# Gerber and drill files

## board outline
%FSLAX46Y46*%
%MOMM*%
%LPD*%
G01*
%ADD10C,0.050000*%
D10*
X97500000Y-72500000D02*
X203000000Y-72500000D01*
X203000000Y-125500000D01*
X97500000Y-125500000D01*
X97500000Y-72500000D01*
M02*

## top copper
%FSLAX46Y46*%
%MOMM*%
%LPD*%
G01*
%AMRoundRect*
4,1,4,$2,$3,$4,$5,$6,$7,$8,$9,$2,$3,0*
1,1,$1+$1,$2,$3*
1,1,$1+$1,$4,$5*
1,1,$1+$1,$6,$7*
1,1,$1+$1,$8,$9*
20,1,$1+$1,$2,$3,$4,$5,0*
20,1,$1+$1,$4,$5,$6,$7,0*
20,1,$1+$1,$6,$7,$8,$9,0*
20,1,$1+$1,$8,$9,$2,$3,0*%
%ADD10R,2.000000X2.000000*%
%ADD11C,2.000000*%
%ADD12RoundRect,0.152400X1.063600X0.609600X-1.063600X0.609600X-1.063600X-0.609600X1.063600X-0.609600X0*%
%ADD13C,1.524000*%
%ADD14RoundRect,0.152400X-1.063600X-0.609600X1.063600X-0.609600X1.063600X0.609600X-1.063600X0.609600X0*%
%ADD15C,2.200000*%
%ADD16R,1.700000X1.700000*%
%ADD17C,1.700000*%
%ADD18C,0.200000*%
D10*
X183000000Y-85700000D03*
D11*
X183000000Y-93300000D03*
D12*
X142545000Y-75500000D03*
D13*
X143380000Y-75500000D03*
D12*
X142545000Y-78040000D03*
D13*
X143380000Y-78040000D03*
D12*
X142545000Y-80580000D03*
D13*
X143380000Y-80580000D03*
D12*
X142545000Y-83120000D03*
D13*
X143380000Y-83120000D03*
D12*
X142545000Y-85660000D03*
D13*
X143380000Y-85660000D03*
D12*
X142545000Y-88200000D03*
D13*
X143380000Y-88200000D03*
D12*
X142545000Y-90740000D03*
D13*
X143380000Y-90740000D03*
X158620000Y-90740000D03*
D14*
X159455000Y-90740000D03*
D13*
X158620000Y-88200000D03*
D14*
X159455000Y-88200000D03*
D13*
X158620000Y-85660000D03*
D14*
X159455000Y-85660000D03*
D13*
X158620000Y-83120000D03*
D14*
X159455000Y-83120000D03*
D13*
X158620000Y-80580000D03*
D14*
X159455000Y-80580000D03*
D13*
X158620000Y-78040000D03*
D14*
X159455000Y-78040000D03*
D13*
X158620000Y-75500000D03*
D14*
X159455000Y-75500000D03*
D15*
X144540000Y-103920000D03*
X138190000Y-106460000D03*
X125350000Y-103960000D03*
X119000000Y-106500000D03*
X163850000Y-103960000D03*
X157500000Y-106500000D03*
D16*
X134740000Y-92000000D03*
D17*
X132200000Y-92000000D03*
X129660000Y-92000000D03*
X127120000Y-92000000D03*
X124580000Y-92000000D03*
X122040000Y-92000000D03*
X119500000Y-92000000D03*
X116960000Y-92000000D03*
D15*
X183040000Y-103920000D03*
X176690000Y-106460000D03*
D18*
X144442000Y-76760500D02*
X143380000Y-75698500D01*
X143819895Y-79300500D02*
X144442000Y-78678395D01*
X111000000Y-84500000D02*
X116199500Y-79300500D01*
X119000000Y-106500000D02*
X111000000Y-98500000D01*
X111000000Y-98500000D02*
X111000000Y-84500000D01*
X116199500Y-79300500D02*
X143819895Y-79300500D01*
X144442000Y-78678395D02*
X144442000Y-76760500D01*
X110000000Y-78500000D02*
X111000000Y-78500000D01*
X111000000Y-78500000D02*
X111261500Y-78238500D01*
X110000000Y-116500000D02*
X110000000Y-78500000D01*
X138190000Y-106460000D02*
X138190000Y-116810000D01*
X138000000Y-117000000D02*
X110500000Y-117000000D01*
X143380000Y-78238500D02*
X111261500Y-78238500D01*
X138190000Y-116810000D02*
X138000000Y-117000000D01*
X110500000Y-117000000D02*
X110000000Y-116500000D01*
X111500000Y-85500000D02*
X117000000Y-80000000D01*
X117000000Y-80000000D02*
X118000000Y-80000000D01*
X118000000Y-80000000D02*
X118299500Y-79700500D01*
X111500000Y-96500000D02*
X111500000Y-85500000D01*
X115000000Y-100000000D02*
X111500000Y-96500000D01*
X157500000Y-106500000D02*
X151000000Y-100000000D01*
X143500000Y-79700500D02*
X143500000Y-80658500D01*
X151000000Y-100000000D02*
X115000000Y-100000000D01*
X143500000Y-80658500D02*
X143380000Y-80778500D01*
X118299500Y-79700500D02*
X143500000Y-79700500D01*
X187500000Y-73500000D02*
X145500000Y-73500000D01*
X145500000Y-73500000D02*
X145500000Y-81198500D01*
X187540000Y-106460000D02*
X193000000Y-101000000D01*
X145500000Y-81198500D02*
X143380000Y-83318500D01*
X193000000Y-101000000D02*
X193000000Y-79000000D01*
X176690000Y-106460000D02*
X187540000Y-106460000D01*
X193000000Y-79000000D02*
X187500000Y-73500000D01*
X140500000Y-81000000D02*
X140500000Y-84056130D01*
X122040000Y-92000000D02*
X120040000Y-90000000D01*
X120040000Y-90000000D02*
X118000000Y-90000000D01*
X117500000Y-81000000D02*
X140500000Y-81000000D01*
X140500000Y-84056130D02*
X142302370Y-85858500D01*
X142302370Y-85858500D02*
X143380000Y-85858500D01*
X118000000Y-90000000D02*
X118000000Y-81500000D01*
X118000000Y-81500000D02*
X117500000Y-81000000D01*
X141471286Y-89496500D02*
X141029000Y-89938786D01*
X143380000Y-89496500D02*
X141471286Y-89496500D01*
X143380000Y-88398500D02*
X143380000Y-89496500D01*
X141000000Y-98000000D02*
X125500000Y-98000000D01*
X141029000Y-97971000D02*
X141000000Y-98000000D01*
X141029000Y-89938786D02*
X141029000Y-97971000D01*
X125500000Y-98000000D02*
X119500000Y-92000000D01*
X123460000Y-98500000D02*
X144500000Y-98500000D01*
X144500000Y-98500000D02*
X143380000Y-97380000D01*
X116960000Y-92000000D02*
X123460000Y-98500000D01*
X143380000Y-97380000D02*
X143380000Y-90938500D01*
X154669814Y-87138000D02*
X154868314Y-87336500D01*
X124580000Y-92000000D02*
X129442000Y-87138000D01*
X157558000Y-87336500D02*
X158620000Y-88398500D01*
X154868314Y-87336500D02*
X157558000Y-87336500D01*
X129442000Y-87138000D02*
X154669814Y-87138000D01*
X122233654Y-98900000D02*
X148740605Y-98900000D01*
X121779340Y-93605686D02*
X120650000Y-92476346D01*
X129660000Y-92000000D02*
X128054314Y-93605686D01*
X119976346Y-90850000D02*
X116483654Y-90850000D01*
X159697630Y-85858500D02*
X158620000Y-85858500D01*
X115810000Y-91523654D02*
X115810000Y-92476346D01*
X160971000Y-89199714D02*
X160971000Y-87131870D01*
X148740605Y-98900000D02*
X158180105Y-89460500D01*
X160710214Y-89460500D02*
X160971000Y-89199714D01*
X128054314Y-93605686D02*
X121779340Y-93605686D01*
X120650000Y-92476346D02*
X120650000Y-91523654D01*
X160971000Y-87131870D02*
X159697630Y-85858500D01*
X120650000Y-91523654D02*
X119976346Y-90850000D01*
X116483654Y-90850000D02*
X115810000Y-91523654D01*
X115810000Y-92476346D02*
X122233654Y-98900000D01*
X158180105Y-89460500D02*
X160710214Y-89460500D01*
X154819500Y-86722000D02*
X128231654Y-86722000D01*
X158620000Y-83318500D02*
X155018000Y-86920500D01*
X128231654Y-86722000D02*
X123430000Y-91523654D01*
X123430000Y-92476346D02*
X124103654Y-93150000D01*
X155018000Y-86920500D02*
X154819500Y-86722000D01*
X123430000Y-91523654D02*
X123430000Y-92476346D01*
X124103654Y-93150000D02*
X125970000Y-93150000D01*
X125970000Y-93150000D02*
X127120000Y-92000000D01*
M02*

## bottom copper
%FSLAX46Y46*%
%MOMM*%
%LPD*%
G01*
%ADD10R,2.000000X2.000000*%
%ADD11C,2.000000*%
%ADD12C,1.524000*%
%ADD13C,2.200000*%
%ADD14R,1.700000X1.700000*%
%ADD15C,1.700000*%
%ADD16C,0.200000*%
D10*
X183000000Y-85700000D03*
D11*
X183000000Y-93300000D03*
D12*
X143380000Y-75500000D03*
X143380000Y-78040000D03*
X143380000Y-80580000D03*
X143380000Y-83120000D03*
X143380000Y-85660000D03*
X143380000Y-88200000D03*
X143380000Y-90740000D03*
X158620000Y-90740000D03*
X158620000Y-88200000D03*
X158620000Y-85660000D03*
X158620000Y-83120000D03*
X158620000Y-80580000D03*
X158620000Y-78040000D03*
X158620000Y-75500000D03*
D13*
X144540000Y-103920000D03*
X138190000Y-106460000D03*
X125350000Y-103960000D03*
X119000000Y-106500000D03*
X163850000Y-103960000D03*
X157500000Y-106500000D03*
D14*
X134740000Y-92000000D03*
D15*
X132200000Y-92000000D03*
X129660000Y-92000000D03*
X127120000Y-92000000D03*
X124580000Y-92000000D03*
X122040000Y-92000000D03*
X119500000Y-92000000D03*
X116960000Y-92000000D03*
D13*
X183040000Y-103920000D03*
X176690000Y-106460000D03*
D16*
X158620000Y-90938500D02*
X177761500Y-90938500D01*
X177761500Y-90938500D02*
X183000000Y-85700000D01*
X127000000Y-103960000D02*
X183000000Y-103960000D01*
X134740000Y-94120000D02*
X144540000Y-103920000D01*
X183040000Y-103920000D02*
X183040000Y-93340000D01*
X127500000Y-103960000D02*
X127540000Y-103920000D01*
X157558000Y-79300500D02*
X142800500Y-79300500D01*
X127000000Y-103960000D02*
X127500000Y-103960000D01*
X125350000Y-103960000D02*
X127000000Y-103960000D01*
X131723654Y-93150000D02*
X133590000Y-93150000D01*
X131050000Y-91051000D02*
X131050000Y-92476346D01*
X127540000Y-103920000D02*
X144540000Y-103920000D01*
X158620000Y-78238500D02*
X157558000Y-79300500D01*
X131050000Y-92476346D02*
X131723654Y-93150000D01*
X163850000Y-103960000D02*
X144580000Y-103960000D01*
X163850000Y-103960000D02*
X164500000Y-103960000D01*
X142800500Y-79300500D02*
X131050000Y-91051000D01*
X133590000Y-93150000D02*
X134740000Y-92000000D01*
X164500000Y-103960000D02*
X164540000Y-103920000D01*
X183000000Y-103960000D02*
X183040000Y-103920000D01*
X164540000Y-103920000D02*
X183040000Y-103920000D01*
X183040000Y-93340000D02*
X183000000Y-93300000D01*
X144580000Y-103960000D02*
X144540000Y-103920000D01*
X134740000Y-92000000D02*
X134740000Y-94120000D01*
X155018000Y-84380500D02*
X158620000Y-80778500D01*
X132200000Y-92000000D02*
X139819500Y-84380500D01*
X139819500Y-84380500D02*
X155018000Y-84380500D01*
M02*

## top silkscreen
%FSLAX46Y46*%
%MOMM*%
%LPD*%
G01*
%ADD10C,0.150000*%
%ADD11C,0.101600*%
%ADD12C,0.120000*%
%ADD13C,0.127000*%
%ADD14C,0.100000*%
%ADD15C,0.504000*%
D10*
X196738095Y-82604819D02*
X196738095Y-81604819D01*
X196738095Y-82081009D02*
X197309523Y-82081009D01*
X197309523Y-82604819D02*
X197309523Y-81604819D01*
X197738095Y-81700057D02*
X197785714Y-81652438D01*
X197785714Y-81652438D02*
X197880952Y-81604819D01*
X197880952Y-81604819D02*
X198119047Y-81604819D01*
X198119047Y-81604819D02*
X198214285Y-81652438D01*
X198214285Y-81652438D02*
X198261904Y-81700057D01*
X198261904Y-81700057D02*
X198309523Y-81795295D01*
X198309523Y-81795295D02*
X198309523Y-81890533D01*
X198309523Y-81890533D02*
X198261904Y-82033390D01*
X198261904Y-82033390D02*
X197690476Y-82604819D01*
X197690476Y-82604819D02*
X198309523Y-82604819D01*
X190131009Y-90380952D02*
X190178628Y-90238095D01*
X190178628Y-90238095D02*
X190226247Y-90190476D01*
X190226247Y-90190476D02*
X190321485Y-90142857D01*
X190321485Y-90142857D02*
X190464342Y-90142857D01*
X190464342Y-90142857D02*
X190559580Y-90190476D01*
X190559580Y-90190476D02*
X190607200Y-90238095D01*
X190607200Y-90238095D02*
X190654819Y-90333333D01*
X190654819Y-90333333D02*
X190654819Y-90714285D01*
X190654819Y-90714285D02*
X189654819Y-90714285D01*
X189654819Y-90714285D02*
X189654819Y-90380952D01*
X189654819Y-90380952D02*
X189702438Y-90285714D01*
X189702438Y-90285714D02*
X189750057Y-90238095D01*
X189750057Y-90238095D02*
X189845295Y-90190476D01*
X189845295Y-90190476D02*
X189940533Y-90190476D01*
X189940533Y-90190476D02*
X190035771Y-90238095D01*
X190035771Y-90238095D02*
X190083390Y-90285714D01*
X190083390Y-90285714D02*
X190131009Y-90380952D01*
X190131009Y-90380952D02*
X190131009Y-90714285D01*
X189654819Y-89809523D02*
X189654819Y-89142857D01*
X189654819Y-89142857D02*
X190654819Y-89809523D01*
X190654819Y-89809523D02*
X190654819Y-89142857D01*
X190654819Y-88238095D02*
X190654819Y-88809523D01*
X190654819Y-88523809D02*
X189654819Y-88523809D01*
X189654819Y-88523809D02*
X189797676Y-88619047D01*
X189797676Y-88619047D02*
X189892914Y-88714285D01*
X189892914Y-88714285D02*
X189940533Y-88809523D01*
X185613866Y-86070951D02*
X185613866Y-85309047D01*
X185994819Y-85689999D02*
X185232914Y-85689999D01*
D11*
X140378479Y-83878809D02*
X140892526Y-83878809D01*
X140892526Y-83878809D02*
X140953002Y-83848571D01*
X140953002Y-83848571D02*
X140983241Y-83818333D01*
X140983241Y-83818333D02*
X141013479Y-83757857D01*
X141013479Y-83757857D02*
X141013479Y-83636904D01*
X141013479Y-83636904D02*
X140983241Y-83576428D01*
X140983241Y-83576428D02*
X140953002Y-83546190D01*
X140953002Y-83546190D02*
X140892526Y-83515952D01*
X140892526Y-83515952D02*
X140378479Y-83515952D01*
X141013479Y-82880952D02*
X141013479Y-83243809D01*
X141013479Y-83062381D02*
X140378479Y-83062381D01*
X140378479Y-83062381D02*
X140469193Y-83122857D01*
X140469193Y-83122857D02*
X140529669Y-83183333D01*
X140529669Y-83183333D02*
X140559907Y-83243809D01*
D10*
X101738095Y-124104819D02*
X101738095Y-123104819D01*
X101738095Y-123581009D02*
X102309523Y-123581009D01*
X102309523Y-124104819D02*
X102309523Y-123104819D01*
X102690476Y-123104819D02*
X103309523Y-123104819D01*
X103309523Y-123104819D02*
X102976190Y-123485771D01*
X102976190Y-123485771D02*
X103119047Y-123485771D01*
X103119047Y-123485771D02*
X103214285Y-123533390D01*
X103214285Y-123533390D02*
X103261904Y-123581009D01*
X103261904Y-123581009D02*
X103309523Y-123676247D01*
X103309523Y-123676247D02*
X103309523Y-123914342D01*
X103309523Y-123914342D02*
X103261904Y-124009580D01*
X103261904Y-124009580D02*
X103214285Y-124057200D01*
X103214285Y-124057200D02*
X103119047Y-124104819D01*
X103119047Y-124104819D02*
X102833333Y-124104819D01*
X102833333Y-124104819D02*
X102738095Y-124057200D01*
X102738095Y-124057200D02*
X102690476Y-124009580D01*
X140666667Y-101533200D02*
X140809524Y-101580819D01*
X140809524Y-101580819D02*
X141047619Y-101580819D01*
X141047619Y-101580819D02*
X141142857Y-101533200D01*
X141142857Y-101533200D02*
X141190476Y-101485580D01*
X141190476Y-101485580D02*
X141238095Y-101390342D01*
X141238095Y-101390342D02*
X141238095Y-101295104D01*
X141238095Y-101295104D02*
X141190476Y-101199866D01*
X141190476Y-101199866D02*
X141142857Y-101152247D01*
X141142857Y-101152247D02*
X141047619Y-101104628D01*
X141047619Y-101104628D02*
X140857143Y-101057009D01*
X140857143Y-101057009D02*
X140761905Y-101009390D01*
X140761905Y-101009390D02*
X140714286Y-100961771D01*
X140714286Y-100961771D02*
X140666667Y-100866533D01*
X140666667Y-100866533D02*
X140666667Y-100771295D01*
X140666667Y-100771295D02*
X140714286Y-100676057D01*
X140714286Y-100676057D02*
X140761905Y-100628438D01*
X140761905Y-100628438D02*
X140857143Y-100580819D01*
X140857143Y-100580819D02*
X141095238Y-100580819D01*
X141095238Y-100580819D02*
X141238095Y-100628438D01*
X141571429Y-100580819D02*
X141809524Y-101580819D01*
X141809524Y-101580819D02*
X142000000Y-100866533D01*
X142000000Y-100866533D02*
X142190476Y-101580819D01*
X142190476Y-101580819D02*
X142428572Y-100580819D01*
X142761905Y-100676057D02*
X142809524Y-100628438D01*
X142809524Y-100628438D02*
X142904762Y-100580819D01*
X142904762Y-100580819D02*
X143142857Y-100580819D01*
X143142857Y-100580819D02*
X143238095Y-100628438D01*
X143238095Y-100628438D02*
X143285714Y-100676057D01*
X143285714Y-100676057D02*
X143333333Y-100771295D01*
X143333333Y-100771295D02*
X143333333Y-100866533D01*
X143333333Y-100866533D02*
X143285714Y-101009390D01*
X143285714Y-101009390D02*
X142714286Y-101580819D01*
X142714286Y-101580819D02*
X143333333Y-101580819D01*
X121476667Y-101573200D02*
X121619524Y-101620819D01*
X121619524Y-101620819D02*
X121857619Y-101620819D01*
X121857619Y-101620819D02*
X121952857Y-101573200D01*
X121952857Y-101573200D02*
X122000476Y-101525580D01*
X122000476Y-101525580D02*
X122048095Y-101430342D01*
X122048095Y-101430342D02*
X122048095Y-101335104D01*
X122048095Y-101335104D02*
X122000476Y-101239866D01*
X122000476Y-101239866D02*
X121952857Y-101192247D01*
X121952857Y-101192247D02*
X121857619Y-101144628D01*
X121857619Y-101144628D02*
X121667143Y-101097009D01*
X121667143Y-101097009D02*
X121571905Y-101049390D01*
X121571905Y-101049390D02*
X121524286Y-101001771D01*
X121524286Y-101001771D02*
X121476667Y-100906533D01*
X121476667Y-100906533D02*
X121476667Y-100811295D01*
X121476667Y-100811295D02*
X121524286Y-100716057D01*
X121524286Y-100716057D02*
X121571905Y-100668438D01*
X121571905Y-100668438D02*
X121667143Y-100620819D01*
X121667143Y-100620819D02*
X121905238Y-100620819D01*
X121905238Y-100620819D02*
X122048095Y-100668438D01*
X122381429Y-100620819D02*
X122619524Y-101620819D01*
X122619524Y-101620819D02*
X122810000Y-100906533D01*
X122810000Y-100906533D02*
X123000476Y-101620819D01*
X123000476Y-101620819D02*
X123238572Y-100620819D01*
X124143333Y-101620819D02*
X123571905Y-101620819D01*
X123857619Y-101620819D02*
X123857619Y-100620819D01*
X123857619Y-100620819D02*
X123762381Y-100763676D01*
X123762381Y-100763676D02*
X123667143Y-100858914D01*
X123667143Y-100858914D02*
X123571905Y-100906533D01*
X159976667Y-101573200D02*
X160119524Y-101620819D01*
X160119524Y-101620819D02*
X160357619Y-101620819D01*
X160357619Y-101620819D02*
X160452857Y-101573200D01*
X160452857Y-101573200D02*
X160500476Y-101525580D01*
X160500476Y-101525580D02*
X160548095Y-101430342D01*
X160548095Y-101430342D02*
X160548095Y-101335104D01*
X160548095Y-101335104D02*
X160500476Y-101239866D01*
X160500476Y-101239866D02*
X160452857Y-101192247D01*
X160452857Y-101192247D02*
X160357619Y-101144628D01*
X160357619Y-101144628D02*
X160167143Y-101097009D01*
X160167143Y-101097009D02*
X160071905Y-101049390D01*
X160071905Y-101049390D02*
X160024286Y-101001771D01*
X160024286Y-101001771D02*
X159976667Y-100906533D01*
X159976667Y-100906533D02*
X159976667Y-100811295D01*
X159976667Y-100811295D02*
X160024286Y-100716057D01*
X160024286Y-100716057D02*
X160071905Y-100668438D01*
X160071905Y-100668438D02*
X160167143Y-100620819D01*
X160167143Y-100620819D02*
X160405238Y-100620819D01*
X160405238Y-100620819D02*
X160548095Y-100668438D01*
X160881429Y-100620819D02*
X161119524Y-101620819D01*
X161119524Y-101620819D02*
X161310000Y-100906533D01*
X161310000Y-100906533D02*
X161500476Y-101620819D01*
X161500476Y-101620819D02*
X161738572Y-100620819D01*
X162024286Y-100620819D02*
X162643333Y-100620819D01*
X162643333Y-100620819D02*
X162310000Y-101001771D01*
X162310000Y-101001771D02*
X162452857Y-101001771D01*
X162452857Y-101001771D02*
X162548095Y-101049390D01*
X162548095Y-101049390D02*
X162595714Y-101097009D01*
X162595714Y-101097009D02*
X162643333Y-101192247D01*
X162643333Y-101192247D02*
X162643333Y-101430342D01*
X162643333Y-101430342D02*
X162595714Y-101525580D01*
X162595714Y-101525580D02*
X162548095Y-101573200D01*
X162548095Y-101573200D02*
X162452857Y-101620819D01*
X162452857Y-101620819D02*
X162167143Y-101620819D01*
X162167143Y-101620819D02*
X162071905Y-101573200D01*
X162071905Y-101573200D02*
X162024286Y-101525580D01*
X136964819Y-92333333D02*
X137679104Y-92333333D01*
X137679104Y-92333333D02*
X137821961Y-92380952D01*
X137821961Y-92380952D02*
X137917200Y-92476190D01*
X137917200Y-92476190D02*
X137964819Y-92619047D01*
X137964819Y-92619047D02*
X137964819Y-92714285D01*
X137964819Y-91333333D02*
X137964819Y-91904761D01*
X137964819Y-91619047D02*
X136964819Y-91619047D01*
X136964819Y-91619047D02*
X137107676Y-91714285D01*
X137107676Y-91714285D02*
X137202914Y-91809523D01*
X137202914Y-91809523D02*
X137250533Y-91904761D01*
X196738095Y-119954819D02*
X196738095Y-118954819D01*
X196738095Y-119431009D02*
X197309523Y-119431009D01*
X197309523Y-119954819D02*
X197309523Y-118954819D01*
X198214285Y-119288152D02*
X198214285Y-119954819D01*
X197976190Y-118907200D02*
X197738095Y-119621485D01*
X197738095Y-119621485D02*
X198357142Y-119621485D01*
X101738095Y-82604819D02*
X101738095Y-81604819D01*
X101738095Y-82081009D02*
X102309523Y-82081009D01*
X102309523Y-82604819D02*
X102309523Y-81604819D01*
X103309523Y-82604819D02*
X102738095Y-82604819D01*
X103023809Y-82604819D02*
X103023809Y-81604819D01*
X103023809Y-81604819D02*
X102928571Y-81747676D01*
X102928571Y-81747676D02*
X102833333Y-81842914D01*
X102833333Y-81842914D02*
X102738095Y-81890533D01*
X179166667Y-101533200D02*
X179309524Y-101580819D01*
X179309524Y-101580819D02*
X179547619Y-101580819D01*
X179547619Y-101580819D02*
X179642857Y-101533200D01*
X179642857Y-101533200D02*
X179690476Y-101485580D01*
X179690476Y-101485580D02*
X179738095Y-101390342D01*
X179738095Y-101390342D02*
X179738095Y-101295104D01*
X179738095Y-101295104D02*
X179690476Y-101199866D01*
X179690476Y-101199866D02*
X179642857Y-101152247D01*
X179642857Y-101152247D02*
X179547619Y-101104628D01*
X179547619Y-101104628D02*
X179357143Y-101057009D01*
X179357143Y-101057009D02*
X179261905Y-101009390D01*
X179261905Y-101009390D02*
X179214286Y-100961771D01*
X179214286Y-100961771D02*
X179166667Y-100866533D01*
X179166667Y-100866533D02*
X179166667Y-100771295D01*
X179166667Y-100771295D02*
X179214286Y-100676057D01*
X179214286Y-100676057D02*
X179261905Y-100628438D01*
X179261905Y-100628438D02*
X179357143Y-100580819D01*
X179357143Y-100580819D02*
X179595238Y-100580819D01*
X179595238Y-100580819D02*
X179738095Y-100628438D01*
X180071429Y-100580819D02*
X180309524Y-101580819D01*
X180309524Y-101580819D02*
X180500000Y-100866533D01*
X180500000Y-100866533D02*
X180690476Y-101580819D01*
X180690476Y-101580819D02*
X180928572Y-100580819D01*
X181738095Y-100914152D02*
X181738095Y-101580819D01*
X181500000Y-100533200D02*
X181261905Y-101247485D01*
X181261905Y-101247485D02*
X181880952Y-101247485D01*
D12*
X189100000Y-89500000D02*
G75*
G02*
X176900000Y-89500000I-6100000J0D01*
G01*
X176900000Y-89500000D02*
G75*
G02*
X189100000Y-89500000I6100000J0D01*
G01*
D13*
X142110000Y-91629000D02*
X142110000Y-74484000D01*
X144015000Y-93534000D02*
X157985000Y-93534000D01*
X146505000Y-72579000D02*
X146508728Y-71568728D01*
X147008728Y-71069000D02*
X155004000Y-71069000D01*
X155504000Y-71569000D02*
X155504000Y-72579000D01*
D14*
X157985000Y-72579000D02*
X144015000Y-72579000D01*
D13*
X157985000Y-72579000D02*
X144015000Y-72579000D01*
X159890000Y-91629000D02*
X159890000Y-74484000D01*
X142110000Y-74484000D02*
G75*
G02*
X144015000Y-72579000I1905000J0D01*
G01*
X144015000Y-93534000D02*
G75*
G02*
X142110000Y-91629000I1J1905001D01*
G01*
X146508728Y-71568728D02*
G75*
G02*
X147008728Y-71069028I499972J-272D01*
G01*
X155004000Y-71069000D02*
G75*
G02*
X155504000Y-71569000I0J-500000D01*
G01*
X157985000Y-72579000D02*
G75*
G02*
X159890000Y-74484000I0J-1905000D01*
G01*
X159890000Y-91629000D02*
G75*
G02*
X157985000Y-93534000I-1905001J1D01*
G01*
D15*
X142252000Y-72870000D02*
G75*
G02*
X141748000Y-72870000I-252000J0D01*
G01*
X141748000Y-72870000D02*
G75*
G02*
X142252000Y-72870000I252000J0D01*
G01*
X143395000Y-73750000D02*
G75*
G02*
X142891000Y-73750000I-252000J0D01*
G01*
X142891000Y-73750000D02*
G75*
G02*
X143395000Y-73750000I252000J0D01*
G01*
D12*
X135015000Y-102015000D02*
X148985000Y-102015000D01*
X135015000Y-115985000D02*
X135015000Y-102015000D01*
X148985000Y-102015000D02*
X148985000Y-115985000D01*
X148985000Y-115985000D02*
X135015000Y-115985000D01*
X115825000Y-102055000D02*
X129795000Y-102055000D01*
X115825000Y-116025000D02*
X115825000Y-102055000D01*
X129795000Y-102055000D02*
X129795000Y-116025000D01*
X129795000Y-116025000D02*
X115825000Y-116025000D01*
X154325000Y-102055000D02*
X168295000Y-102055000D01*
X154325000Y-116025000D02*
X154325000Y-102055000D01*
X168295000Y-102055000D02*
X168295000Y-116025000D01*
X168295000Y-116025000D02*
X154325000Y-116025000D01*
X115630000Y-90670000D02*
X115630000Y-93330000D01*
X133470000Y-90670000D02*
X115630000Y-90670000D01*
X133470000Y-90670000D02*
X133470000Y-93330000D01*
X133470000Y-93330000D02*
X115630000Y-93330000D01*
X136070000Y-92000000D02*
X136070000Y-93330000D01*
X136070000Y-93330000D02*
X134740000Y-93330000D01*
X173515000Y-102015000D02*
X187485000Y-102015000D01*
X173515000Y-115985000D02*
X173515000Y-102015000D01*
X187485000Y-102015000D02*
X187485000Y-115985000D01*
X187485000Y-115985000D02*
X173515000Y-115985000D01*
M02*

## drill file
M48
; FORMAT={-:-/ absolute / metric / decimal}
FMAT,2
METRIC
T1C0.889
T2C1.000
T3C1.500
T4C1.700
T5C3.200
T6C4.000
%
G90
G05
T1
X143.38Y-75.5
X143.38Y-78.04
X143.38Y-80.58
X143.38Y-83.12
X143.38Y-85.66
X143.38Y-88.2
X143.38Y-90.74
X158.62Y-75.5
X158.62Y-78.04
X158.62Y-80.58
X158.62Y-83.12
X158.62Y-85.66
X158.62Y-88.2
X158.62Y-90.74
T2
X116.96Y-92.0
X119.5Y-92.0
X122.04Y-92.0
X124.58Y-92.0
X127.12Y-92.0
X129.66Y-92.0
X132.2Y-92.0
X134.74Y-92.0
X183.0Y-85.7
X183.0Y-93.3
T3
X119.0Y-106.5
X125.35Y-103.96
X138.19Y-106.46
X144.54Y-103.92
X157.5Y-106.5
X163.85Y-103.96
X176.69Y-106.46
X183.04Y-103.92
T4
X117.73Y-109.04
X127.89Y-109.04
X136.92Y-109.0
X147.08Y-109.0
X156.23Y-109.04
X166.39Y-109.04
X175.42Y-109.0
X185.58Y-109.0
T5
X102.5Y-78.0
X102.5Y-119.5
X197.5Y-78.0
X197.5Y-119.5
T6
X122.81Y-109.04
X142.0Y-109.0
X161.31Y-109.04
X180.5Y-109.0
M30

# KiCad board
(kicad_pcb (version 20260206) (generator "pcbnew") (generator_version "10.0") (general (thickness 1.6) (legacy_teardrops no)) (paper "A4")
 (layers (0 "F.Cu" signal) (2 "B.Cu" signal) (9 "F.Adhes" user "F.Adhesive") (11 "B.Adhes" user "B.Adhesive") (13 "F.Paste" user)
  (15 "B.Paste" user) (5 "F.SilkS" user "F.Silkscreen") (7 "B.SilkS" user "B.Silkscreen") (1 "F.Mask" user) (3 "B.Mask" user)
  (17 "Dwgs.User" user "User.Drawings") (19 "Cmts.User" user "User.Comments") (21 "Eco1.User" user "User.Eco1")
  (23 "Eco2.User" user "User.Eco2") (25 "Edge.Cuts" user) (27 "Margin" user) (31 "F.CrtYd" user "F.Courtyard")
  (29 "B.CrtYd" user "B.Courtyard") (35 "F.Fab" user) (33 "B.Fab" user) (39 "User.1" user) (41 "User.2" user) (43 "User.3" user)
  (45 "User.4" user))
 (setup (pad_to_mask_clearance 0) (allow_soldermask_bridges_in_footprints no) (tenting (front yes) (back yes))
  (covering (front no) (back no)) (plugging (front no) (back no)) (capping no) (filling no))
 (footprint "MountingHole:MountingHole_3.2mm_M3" (layer "F.Cu") (at 197.5 78 180)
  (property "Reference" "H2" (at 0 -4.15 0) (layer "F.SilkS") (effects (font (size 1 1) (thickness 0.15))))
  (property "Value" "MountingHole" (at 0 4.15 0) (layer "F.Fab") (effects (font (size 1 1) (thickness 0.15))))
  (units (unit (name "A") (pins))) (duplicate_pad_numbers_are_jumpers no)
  (pad "" np_thru_hole circle (at 0 0 180) (size 3.2 3.2) (drill 3.2) (layers "*.Cu" "*.Mask")))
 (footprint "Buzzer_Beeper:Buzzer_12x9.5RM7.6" (layer "F.Cu") (at 183 85.7 -90)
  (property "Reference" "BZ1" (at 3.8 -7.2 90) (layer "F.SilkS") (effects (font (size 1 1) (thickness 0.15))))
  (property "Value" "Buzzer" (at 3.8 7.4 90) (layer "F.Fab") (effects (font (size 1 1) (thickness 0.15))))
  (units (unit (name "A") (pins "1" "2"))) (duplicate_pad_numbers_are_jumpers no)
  (fp_circle (center 3.8 0) (end 9.9 0) (stroke (width 0.12) (type solid)) (fill no) (layer "F.SilkS"))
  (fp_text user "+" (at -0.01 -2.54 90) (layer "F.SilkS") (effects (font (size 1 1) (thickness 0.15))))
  (pad "1" thru_hole rect (at 0 0 270) (size 2 2) (drill 1) (layers "*.Cu" "*.Mask") (remove_unused_layers no) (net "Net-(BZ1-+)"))
  (pad "2" thru_hole circle (at 7.6 0 270) (size 2 2) (drill 1) (layers "*.Cu" "*.Mask") (remove_unused_layers no) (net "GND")))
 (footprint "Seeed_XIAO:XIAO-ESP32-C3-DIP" (layer "F.Cu") (at 151 83.12 90)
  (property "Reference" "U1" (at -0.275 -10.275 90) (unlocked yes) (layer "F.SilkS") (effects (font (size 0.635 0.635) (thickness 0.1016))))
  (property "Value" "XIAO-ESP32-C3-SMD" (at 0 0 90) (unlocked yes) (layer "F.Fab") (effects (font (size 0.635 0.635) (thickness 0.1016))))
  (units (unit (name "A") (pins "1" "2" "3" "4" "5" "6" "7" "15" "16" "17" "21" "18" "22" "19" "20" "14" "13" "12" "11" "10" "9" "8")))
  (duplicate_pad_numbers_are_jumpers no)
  (fp_line (start -8.509 -8.89) (end 8.636 -8.89) (stroke (width 0.127) (type solid)) (layer "F.SilkS"))
  (fp_line (start -10.414 -6.985) (end -10.414 6.985) (stroke (width 0.127) (type solid)) (layer "F.SilkS"))
  (fp_line (start 10.541 -4.495) (end 11.551272 -4.491272) (stroke (width 0.127) (type solid)) (layer "F.SilkS"))
  (fp_line (start 12.051 -3.991272) (end 12.051 4.004) (stroke (width 0.127) (type solid)) (layer "F.SilkS"))
  (fp_line (start 11.551 4.504) (end 10.541 4.504) (stroke (width 0.127) (type solid)) (layer "F.SilkS"))
  (fp_line (start 10.541 6.985) (end 10.541 -6.985) (stroke (width 0.1) (type solid)) (layer "F.SilkS"))
  (fp_line (start 10.541 6.985) (end 10.541 -6.985) (stroke (width 0.127) (type solid)) (layer "F.SilkS"))
  (fp_line (start -8.509 8.89) (end 8.636 8.89) (stroke (width 0.127) (type solid)) (layer "F.SilkS"))
  (fp_arc (start 8.636 -8.89) (mid 9.983038 -8.332038) (end 10.541 -6.985) (stroke (width 0.127) (type solid)) (layer "F.SilkS"))
  (fp_arc (start -10.414 -6.985) (mid -9.856038 -8.332038) (end -8.509 -8.89) (stroke (width 0.127) (type solid)) (layer "F.SilkS"))
  (fp_arc (start 11.551272 -4.491272) (mid 11.904644 -4.344724) (end 12.051 -3.991272) (stroke (width 0.127) (type default))
   (layer "F.SilkS"))
  (fp_arc (start 12.051 4.004) (mid 11.904553 4.357553) (end 11.551 4.504) (stroke (width 0.127) (type default)) (layer "F.SilkS"))
  (fp_arc (start 10.541 6.985) (mid 9.983038 8.332038) (end 8.636 8.89) (stroke (width 0.127) (type solid)) (layer "F.SilkS"))
  (fp_arc (start -8.509 8.89) (mid -9.856038 8.332038) (end -10.414 6.985) (stroke (width 0.127) (type solid)) (layer "F.SilkS"))
  (fp_circle (center 10.25 -9) (end 10.504 -9) (stroke (width 0.5) (type solid)) (fill yes) (layer "F.SilkS"))
  (fp_circle (center 9.37 -7.857) (end 9.624 -7.857) (stroke (width 0.5) (type solid)) (fill yes) (layer "F.SilkS"))
  (pad "1" smd roundrect (at 7.62 -8.455 180) (size 2.432 1.524) (layers "F.Cu" "F.Mask") (roundrect_rratio 0.1) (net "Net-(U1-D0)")
   (thermal_bridge_angle 45))
  (pad "1" thru_hole circle (at 7.62 -7.62 180) (size 1.524 1.524) (drill 0.889) (layers "*.Cu" "*.Mask") (remove_unused_layers no)
   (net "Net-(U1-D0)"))
  (pad "2" smd roundrect (at 5.08 -8.455 180) (size 2.432 1.524) (layers "F.Cu" "F.Mask") (roundrect_rratio 0.1) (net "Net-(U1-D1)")
   (thermal_bridge_angle 45))
  (pad "2" thru_hole circle (at 5.08 -7.62 180) (size 1.524 1.524) (drill 0.889) (layers "*.Cu" "*.Mask") (remove_unused_layers no)
   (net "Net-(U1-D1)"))
  (pad "3" smd roundrect (at 2.54 -8.455 180) (size 2.432 1.524) (layers "F.Cu" "F.Mask") (roundrect_rratio 0.1) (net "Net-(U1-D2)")
   (thermal_bridge_angle 45))
  (pad "3" thru_hole circle (at 2.54 -7.62 180) (size 1.524 1.524) (drill 0.889) (layers "*.Cu" "*.Mask") (remove_unused_layers no)
   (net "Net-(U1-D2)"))
  (pad "4" smd roundrect (at 0 -8.455 180) (size 2.432 1.524) (layers "F.Cu" "F.Mask") (roundrect_rratio 0.1) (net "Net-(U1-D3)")
   (thermal_bridge_angle 45))
  (pad "4" thru_hole circle (at 0 -7.62 180) (size 1.524 1.524) (drill 0.889) (layers "*.Cu" "*.Mask") (remove_unused_layers no)
   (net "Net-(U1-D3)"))
  (pad "5" smd roundrect (at -2.54 -8.455 180) (size 2.432 1.524) (layers "F.Cu" "F.Mask") (roundrect_rratio 0.1) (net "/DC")
   (thermal_bridge_angle 45))
  (pad "5" thru_hole circle (at -2.54 -7.62 180) (size 1.524 1.524) (drill 0.889) (layers "*.Cu" "*.Mask") (remove_unused_layers no)
   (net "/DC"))
  (pad "6" smd roundrect (at -5.08 -8.455 180) (size 2.432 1.524) (layers "F.Cu" "F.Mask") (roundrect_rratio 0.1) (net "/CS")
   (thermal_bridge_angle 45))
  (pad "6" thru_hole circle (at -5.08 -7.62 180) (size 1.524 1.524) (drill 0.889) (layers "*.Cu" "*.Mask") (remove_unused_layers no)
   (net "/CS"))
  (pad "7" smd roundrect (at -7.62 -8.455 180) (size 2.432 1.524) (layers "F.Cu" "F.Mask") (roundrect_rratio 0.1) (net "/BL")
   (thermal_bridge_angle 45))
  (pad "7" thru_hole circle (at -7.62 -7.62 180) (size 1.524 1.524) (drill 0.889) (layers "*.Cu" "*.Mask") (remove_unused_layers no)
   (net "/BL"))
  (pad "8" thru_hole circle (at -7.62 7.62) (size 1.524 1.524) (drill 0.889) (layers "*.Cu" "*.Mask") (remove_unused_layers no)
   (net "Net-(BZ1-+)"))
  (pad "8" smd roundrect (at -7.62 8.455) (size 2.432 1.524) (layers "F.Cu" "F.Mask") (roundrect_rratio 0.1) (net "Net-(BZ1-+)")
   (thermal_bridge_angle 45))
  (pad "9" thru_hole circle (at -5.08 7.62) (size 1.524 1.524) (drill 0.889) (layers "*.Cu" "*.Mask") (remove_unused_layers no) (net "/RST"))
  (pad "9" smd roundrect (at -5.08 8.455) (size 2.432 1.524) (layers "F.Cu" "F.Mask") (roundrect_rratio 0.1) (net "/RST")
   (thermal_bridge_angle 45))
  (pad "10" thru_hole circle (at -2.54 7.62) (size 1.524 1.524) (drill 0.889) (layers "*.Cu" "*.Mask") (remove_unused_layers no)
   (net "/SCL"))
  (pad "10" smd roundrect (at -2.54 8.455) (size 2.432 1.524) (layers "F.Cu" "F.Mask") (roundrect_rratio 0.1) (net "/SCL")
   (thermal_bridge_angle 45))
  (pad "11" thru_hole circle (at 0 7.62) (size 1.524 1.524) (drill 0.889) (layers "*.Cu" "*.Mask") (remove_unused_layers no) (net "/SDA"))
  (pad "11" smd roundrect (at 0 8.455) (size 2.432 1.524) (layers "F.Cu" "F.Mask") (roundrect_rratio 0.1) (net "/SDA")
   (thermal_bridge_angle 45))
  (pad "12" thru_hole circle (at 2.54 7.62) (size 1.524 1.524) (drill 0.889) (layers "*.Cu" "*.Mask") (remove_unused_layers no)
   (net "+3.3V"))
  (pad "12" smd roundrect (at 2.54 8.455) (size 2.432 1.524) (layers "F.Cu" "F.Mask") (roundrect_rratio 0.1) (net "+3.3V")
   (thermal_bridge_angle 45))
  (pad "13" thru_hole circle (at 5.08 7.62) (size 1.524 1.524) (drill 0.889) (layers "*.Cu" "*.Mask") (remove_unused_layers no) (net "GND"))
  (pad "13" smd roundrect (at 5.08 8.455) (size 2.432 1.524) (layers "F.Cu" "F.Mask") (roundrect_rratio 0.1) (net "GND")
   (thermal_bridge_angle 45))
  (pad "14" thru_hole circle (at 7.62 7.62) (size 1.524 1.524) (drill 0.889) (layers "*.Cu" "*.Mask") (remove_unused_layers no)
   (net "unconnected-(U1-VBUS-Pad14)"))
  (pad "14" smd roundrect (at 7.62 8.455) (size 2.432 1.524) (layers "F.Cu" "F.Mask") (roundrect_rratio 0.1)
   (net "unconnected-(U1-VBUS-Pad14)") (thermal_bridge_angle 45)))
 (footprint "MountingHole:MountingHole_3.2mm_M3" (layer "F.Cu") (at 102.5 119.5 180)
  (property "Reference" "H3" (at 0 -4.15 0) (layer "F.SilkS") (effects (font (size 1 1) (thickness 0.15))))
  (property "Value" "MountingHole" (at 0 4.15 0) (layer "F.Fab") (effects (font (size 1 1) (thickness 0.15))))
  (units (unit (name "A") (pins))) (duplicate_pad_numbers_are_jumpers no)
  (pad "" np_thru_hole circle (at 0 0 180) (size 3.2 3.2) (drill 3.2) (layers "*.Cu" "*.Mask")))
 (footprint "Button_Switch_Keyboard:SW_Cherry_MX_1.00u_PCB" (layer "F.Cu") (at 144.54 103.92)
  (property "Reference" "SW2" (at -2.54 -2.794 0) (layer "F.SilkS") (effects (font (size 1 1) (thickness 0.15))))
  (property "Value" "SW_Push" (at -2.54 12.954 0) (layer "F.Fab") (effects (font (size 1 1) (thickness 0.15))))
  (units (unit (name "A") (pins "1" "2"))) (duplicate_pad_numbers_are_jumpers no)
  (fp_line (start -9.525 -1.905) (end 4.445 -1.905) (stroke (width 0.12) (type solid)) (layer "F.SilkS"))
  (fp_line (start -9.525 12.065) (end -9.525 -1.905) (stroke (width 0.12) (type solid)) (layer "F.SilkS"))
  (fp_line (start 4.445 -1.905) (end 4.445 12.065) (stroke (width 0.12) (type solid)) (layer "F.SilkS"))
  (fp_line (start 4.445 12.065) (end -9.525 12.065) (stroke (width 0.12) (type solid)) (layer "F.SilkS"))
  (pad "" np_thru_hole circle (at -7.62 5.08) (size 1.7 1.7) (drill 1.7) (layers "*.Cu" "*.Mask"))
  (pad "" np_thru_hole circle (at -2.54 5.08) (size 4 4) (drill 4) (layers "*.Cu" "*.Mask"))
  (pad "" np_thru_hole circle (at 2.54 5.08) (size 1.7 1.7) (drill 1.7) (layers "*.Cu" "*.Mask"))
  (pad "1" thru_hole circle (at 0 0) (size 2.2 2.2) (drill 1.5) (layers "*.Cu" "*.Mask") (remove_unused_layers no) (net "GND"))
  (pad "2" thru_hole circle (at -6.35 2.54) (size 2.2 2.2) (drill 1.5) (layers "*.Cu" "*.Mask") (remove_unused_layers no)
   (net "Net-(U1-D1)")))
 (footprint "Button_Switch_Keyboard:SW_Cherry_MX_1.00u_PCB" (layer "F.Cu") (at 125.35 103.96)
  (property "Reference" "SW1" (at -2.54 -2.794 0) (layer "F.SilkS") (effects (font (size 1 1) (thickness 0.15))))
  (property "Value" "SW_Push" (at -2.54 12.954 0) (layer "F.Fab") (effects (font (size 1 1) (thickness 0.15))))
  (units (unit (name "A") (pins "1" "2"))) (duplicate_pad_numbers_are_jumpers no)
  (fp_line (start -9.525 -1.905) (end 4.445 -1.905) (stroke (width 0.12) (type solid)) (layer "F.SilkS"))
  (fp_line (start -9.525 12.065) (end -9.525 -1.905) (stroke (width 0.12) (type solid)) (layer "F.SilkS"))
  (fp_line (start 4.445 -1.905) (end 4.445 12.065) (stroke (width 0.12) (type solid)) (layer "F.SilkS"))
  (fp_line (start 4.445 12.065) (end -9.525 12.065) (stroke (width 0.12) (type solid)) (layer "F.SilkS"))
  (pad "" np_thru_hole circle (at -7.62 5.08) (size 1.7 1.7) (drill 1.7) (layers "*.Cu" "*.Mask"))
  (pad "" np_thru_hole circle (at -2.54 5.08) (size 4 4) (drill 4) (layers "*.Cu" "*.Mask"))
  (pad "" np_thru_hole circle (at 2.54 5.08) (size 1.7 1.7) (drill 1.7) (layers "*.Cu" "*.Mask"))
  (pad "1" thru_hole circle (at 0 0) (size 2.2 2.2) (drill 1.5) (layers "*.Cu" "*.Mask") (remove_unused_layers no) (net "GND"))
  (pad "2" thru_hole circle (at -6.35 2.54) (size 2.2 2.2) (drill 1.5) (layers "*.Cu" "*.Mask") (remove_unused_layers no)
   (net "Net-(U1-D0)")))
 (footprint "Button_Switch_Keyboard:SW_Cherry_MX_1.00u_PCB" (layer "F.Cu") (at 163.85 103.96)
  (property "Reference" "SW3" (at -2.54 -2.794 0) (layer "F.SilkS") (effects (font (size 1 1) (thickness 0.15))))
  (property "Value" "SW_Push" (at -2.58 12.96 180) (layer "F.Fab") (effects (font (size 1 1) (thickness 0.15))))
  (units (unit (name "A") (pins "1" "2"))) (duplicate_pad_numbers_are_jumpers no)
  (fp_line (start -9.525 -1.905) (end 4.445 -1.905) (stroke (width 0.12) (type solid)) (layer "F.SilkS"))
  (fp_line (start -9.525 12.065) (end -9.525 -1.905) (stroke (width 0.12) (type solid)) (layer "F.SilkS"))
  (fp_line (start 4.445 -1.905) (end 4.445 12.065) (stroke (width 0.12) (type solid)) (layer "F.SilkS"))
  (fp_line (start 4.445 12.065) (end -9.525 12.065) (stroke (width 0.12) (type solid)) (layer "F.SilkS"))
  (pad "" np_thru_hole circle (at -7.62 5.08) (size 1.7 1.7) (drill 1.7) (layers "*.Cu" "*.Mask"))
  (pad "" np_thru_hole circle (at -2.54 5.08) (size 4 4) (drill 4) (layers "*.Cu" "*.Mask"))
  (pad "" np_thru_hole circle (at 2.54 5.08) (size 1.7 1.7) (drill 1.7) (layers "*.Cu" "*.Mask"))
  (pad "1" thru_hole circle (at 0 0) (size 2.2 2.2) (drill 1.5) (layers "*.Cu" "*.Mask") (remove_unused_layers no) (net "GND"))
  (pad "2" thru_hole circle (at -6.35 2.54) (size 2.2 2.2) (drill 1.5) (layers "*.Cu" "*.Mask") (remove_unused_layers no)
   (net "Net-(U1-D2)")))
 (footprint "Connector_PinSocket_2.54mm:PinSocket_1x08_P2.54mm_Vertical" (layer "F.Cu") (at 134.74 92 -90)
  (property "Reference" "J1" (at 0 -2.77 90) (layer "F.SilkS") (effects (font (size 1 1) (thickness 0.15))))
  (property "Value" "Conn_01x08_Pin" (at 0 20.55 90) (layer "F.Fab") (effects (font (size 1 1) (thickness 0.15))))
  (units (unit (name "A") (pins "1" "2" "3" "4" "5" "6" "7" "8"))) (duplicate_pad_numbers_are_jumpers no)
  (fp_line (start -1.33 19.11) (end 1.33 19.11) (stroke (width 0.12) (type solid)) (layer "F.SilkS"))
  (fp_line (start -1.33 1.27) (end -1.33 19.11) (stroke (width 0.12) (type solid)) (layer "F.SilkS"))
  (fp_line (start -1.33 1.27) (end 1.33 1.27) (stroke (width 0.12) (type solid)) (layer "F.SilkS"))
  (fp_line (start 1.33 1.27) (end 1.33 19.11) (stroke (width 0.12) (type solid)) (layer "F.SilkS"))
  (fp_line (start 0 -1.33) (end 1.33 -1.33) (stroke (width 0.12) (type solid)) (layer "F.SilkS"))
  (fp_line (start 1.33 -1.33) (end 1.33 0) (stroke (width 0.12) (type solid)) (layer "F.SilkS"))
  (pad "1" thru_hole rect (at 0 0 270) (size 1.7 1.7) (drill 1) (layers "*.Cu" "*.Mask") (remove_unused_layers no) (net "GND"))
  (pad "2" thru_hole circle (at 0 2.54 270) (size 1.7 1.7) (drill 1) (layers "*.Cu" "*.Mask") (remove_unused_layers no) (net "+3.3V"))
  (pad "3" thru_hole circle (at 0 5.08 270) (size 1.7 1.7) (drill 1) (layers "*.Cu" "*.Mask") (remove_unused_layers no) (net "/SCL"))
  (pad "4" thru_hole circle (at 0 7.62 270) (size 1.7 1.7) (drill 1) (layers "*.Cu" "*.Mask") (remove_unused_layers no) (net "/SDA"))
  (pad "5" thru_hole circle (at 0 10.16 270) (size 1.7 1.7) (drill 1) (layers "*.Cu" "*.Mask") (remove_unused_layers no) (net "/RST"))
  (pad "6" thru_hole circle (at 0 12.7 270) (size 1.7 1.7) (drill 1) (layers "*.Cu" "*.Mask") (remove_unused_layers no) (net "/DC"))
  (pad "7" thru_hole circle (at 0 15.24 270) (size 1.7 1.7) (drill 1) (layers "*.Cu" "*.Mask") (remove_unused_layers no) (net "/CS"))
  (pad "8" thru_hole circle (at 0 17.78 270) (size 1.7 1.7) (drill 1) (layers "*.Cu" "*.Mask") (remove_unused_layers no) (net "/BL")))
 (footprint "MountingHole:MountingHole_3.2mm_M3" (layer "F.Cu") (at 197.5 119.5 180)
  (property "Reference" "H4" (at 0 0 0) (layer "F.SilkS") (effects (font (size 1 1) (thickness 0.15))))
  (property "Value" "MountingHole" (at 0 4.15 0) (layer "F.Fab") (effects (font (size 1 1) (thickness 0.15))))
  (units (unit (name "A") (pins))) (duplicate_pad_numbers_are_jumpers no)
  (pad "" np_thru_hole circle (at 0 0 180) (size 3.2 3.2) (drill 3.2) (layers "*.Cu" "*.Mask")))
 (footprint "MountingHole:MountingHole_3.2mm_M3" (layer "F.Cu") (at 102.5 78 180)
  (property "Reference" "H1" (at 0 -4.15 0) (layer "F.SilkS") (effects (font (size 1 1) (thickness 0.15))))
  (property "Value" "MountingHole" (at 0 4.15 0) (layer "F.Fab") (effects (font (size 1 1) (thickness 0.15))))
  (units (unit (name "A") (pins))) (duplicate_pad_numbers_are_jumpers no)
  (pad "" np_thru_hole circle (at 0 0 180) (size 3.2 3.2) (drill 3.2) (layers "*.Cu" "*.Mask")))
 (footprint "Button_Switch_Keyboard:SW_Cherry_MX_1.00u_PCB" (layer "F.Cu") (at 183.04 103.92)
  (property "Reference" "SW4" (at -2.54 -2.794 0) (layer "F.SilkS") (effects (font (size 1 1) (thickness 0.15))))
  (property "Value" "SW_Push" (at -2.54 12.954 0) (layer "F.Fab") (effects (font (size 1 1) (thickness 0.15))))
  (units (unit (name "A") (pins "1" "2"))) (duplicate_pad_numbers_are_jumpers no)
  (fp_line (start -9.525 -1.905) (end 4.445 -1.905) (stroke (width 0.12) (type solid)) (layer "F.SilkS"))
  (fp_line (start -9.525 12.065) (end -9.525 -1.905) (stroke (width 0.12) (type solid)) (layer "F.SilkS"))
  (fp_line (start 4.445 -1.905) (end 4.445 12.065) (stroke (width 0.12) (type solid)) (layer "F.SilkS"))
  (fp_line (start 4.445 12.065) (end -9.525 12.065) (stroke (width 0.12) (type solid)) (layer "F.SilkS"))
  (pad "" np_thru_hole circle (at -7.62 5.08) (size 1.7 1.7) (drill 1.7) (layers "*.Cu" "*.Mask"))
  (pad "" np_thru_hole circle (at -2.54 5.08) (size 4 4) (drill 4) (layers "*.Cu" "*.Mask"))
  (pad "" np_thru_hole circle (at 2.54 5.08) (size 1.7 1.7) (drill 1.7) (layers "*.Cu" "*.Mask"))
  (pad "1" thru_hole circle (at 0 0) (size 2.2 2.2) (drill 1.5) (layers "*.Cu" "*.Mask") (remove_unused_layers no) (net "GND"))
  (pad "2" thru_hole circle (at -6.35 2.54) (size 2.2 2.2) (drill 1.5) (layers "*.Cu" "*.Mask") (remove_unused_layers no)
   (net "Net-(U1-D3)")))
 (gr_rect (start 97.5 72.5) (end 203 125.5) (stroke (width 0.05) (type default)) (fill no) (layer "Edge.Cuts"))
 (segment (start 158.62 90.9385) (end 177.7615 90.9385) (width 0.2) (layer "B.Cu") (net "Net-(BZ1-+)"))
 (segment (start 177.7615 90.9385) (end 183 85.7) (width 0.2) (layer "B.Cu") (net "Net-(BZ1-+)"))
 (segment (start 127 103.96) (end 183 103.96) (width 0.2) (layer "B.Cu") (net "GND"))
 (segment (start 134.74 94.12) (end 144.54 103.92) (width 0.2) (layer "B.Cu") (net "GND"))
 (segment (start 183.04 103.92) (end 183.04 93.34) (width 0.2) (layer "B.Cu") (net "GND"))
 (segment (start 127.5 103.96) (end 127.54 103.92) (width 0.2) (layer "B.Cu") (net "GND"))
 (segment (start 157.558 79.3005) (end 142.8005 79.3005) (width 0.2) (layer "B.Cu") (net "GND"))
 (segment (start 127 103.96) (end 127.5 103.96) (width 0.2) (layer "B.Cu") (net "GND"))
 (segment (start 125.35 103.96) (end 127 103.96) (width 0.2) (layer "B.Cu") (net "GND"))
 (segment (start 131.723654 93.15) (end 133.59 93.15) (width 0.2) (layer "B.Cu") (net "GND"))
 (segment (start 131.05 91.051) (end 131.05 92.476346) (width 0.2) (layer "B.Cu") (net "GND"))
 (segment (start 127.54 103.92) (end 144.54 103.92) (width 0.2) (layer "B.Cu") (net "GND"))
 (segment (start 158.62 78.2385) (end 157.558 79.3005) (width 0.2) (layer "B.Cu") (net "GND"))
 (segment (start 131.05 92.476346) (end 131.723654 93.15) (width 0.2) (layer "B.Cu") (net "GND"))
 (segment (start 163.85 103.96) (end 144.58 103.96) (width 0.2) (layer "B.Cu") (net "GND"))
 (segment (start 163.85 103.96) (end 164.5 103.96) (width 0.2) (layer "B.Cu") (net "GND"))
 (segment (start 142.8005 79.3005) (end 131.05 91.051) (width 0.2) (layer "B.Cu") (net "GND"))
 (segment (start 133.59 93.15) (end 134.74 92) (width 0.2) (layer "B.Cu") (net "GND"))
 (segment (start 164.5 103.96) (end 164.54 103.92) (width 0.2) (layer "B.Cu") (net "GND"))
 (segment (start 183 103.96) (end 183.04 103.92) (width 0.2) (layer "B.Cu") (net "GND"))
 (segment (start 164.54 103.92) (end 183.04 103.92) (width 0.2) (layer "B.Cu") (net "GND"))
 (segment (start 183.04 93.34) (end 183 93.3) (width 0.2) (layer "B.Cu") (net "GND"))
 (segment (start 144.58 103.96) (end 144.54 103.92) (width 0.2) (layer "B.Cu") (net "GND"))
 (segment (start 134.74 92) (end 134.74 94.12) (width 0.2) (layer "B.Cu") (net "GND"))
 (segment (start 144.442 76.7605) (end 143.38 75.6985) (width 0.2) (layer "F.Cu") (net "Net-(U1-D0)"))
 (segment (start 143.819895 79.3005) (end 144.442 78.678395) (width 0.2) (layer "F.Cu") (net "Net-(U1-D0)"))
 (segment (start 111 84.5) (end 116.1995 79.3005) (width 0.2) (layer "F.Cu") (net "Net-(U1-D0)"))
 (segment (start 119 106.5) (end 111 98.5) (width 0.2) (layer "F.Cu") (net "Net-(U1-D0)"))
 (segment (start 111 98.5) (end 111 84.5) (width 0.2) (layer "F.Cu") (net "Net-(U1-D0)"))
 (segment (start 116.1995 79.3005) (end 143.819895 79.3005) (width 0.2) (layer "F.Cu") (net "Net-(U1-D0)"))
 (segment (start 144.442 78.678395) (end 144.442 76.7605) (width 0.2) (layer "F.Cu") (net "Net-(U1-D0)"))
 (segment (start 110 78.5) (end 111 78.5) (width 0.2) (layer "F.Cu") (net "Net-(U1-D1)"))
 (segment (start 111 78.5) (end 111.2615 78.2385) (width 0.2) (layer "F.Cu") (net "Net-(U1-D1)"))
 (segment (start 110 116.5) (end 110 78.5) (width 0.2) (layer "F.Cu") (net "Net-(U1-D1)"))
 (segment (start 138.19 106.46) (end 138.19 116.81) (width 0.2) (layer "F.Cu") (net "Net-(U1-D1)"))
 (segment (start 138 117) (end 110.5 117) (width 0.2) (layer "F.Cu") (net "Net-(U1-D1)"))
 (segment (start 143.38 78.2385) (end 111.2615 78.2385) (width 0.2) (layer "F.Cu") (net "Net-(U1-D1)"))
 (segment (start 138.19 116.81) (end 138 117) (width 0.2) (layer "F.Cu") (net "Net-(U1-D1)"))
 (segment (start 110.5 117) (end 110 116.5) (width 0.2) (layer "F.Cu") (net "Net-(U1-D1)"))
 (segment (start 111.5 85.5) (end 117 80) (width 0.2) (layer "F.Cu") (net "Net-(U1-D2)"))
 (segment (start 117 80) (end 118 80) (width 0.2) (layer "F.Cu") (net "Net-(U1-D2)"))
 (segment (start 118 80) (end 118.2995 79.7005) (width 0.2) (layer "F.Cu") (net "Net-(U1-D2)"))
 (segment (start 111.5 96.5) (end 111.5 85.5) (width 0.2) (layer "F.Cu") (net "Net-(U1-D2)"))
 (segment (start 115 100) (end 111.5 96.5) (width 0.2) (layer "F.Cu") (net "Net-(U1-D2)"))
 (segment (start 157.5 106.5) (end 151 100) (width 0.2) (layer "F.Cu") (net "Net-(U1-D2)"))
 (segment (start 143.5 79.7005) (end 143.5 80.6585) (width 0.2) (layer "F.Cu") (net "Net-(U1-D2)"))
 (segment (start 151 100) (end 115 100) (width 0.2) (layer "F.Cu") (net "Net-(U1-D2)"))
 (segment (start 143.5 80.6585) (end 143.38 80.7785) (width 0.2) (layer "F.Cu") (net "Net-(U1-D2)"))
 (segment (start 118.2995 79.7005) (end 143.5 79.7005) (width 0.2) (layer "F.Cu") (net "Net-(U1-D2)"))
 (segment (start 187.5 73.5) (end 145.5 73.5) (width 0.2) (layer "F.Cu") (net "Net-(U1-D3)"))
 (segment (start 145.5 73.5) (end 145.5 81.1985) (width 0.2) (layer "F.Cu") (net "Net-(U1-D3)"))
 (segment (start 187.54 106.46) (end 193 101) (width 0.2) (layer "F.Cu") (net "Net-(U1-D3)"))
 (segment (start 145.5 81.1985) (end 143.38 83.3185) (width 0.2) (layer "F.Cu") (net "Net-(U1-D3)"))
 (segment (start 193 101) (end 193 79) (width 0.2) (layer "F.Cu") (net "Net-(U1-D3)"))
 (segment (start 176.69 106.46) (end 187.54 106.46) (width 0.2) (layer "F.Cu") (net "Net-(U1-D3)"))
 (segment (start 193 79) (end 187.5 73.5) (width 0.2) (layer "F.Cu") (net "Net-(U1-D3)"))
 (segment (start 140.5 81) (end 140.5 84.05613) (width 0.2) (layer "F.Cu") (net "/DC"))
 (segment (start 122.04 92) (end 120.04 90) (width 0.2) (layer "F.Cu") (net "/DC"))
 (segment (start 120.04 90) (end 118 90) (width 0.2) (layer "F.Cu") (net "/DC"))
 (segment (start 117.5 81) (end 140.5 81) (width 0.2) (layer "F.Cu") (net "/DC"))
 (segment (start 140.5 84.05613) (end 142.30237 85.8585) (width 0.2) (layer "F.Cu") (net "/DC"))
 (segment (start 142.30237 85.8585) (end 143.38 85.8585) (width 0.2) (layer "F.Cu") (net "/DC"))
 (segment (start 118 90) (end 118 81.5) (width 0.2) (layer "F.Cu") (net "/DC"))
 (segment (start 118 81.5) (end 117.5 81) (width 0.2) (layer "F.Cu") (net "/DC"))
 (segment (start 141.471286 89.4965) (end 141.029 89.938786) (width 0.2) (layer "F.Cu") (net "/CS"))
 (segment (start 143.38 89.4965) (end 141.471286 89.4965) (width 0.2) (layer "F.Cu") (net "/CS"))
 (segment (start 143.38 88.3985) (end 143.38 89.4965) (width 0.2) (layer "F.Cu") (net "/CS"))
 (segment (start 141 98) (end 125.5 98) (width 0.2) (layer "F.Cu") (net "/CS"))
 (segment (start 141.029 97.971) (end 141 98) (width 0.2) (layer "F.Cu") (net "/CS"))
 (segment (start 141.029 89.938786) (end 141.029 97.971) (width 0.2) (layer "F.Cu") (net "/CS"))
 (segment (start 125.5 98) (end 119.5 92) (width 0.2) (layer "F.Cu") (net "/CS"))
 (segment (start 123.46 98.5) (end 144.5 98.5) (width 0.2) (layer "F.Cu") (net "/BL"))
 (segment (start 144.5 98.5) (end 143.38 97.38) (width 0.2) (layer "F.Cu") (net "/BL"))
 (segment (start 116.96 92) (end 123.46 98.5) (width 0.2) (layer "F.Cu") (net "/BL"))
 (segment (start 143.38 97.38) (end 143.38 90.9385) (width 0.2) (layer "F.Cu") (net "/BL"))
 (segment (start 154.669814 87.138) (end 154.868314 87.3365) (width 0.2) (layer "F.Cu") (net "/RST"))
 (segment (start 124.58 92) (end 129.442 87.138) (width 0.2) (layer "F.Cu") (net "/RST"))
 (segment (start 157.558 87.3365) (end 158.62 88.3985) (width 0.2) (layer "F.Cu") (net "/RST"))
 (segment (start 154.868314 87.3365) (end 157.558 87.3365) (width 0.2) (layer "F.Cu") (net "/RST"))
 (segment (start 129.442 87.138) (end 154.669814 87.138) (width 0.2) (layer "F.Cu") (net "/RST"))
 (segment (start 122.233654 98.9) (end 148.740605 98.9) (width 0.2) (layer "F.Cu") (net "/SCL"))
 (segment (start 121.77934 93.605686) (end 120.65 92.476346) (width 0.2) (layer "F.Cu") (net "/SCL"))
 (segment (start 129.66 92) (end 128.054314 93.605686) (width 0.2) (layer "F.Cu") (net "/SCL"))
 (segment (start 119.976346 90.85) (end 116.483654 90.85) (width 0.2) (layer "F.Cu") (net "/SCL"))
 (segment (start 159.69763 85.8585) (end 158.62 85.8585) (width 0.2) (layer "F.Cu") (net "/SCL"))
 (segment (start 115.81 91.523654) (end 115.81 92.476346) (width 0.2) (layer "F.Cu") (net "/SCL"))
 (segment (start 160.971 89.199714) (end 160.971 87.13187) (width 0.2) (layer "F.Cu") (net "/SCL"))
 (segment (start 148.740605 98.9) (end 158.180105 89.4605) (width 0.2) (layer "F.Cu") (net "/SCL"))
 (segment (start 160.710214 89.4605) (end 160.971 89.199714) (width 0.2) (layer "F.Cu") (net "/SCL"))
 (segment (start 128.054314 93.605686) (end 121.77934 93.605686) (width 0.2) (layer "F.Cu") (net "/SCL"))
 (segment (start 120.65 92.476346) (end 120.65 91.523654) (width 0.2) (layer "F.Cu") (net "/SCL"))
 (segment (start 160.971 87.13187) (end 159.69763 85.8585) (width 0.2) (layer "F.Cu") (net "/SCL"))
 (segment (start 120.65 91.523654) (end 119.976346 90.85) (width 0.2) (layer "F.Cu") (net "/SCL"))
 (segment (start 116.483654 90.85) (end 115.81 91.523654) (width 0.2) (layer "F.Cu") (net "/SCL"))
 (segment (start 115.81 92.476346) (end 122.233654 98.9) (width 0.2) (layer "F.Cu") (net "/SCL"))
 (segment (start 158.180105 89.4605) (end 160.710214 89.4605) (width 0.2) (layer "F.Cu") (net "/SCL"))
 (segment (start 154.8195 86.722) (end 128.231654 86.722) (width 0.2) (layer "F.Cu") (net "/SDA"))
 (segment (start 158.62 83.3185) (end 155.018 86.9205) (width 0.2) (layer "F.Cu") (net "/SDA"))
 (segment (start 128.231654 86.722) (end 123.43 91.523654) (width 0.2) (layer "F.Cu") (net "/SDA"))
 (segment (start 123.43 92.476346) (end 124.103654 93.15) (width 0.2) (layer "F.Cu") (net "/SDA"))
 (segment (start 155.018 86.9205) (end 154.8195 86.722) (width 0.2) (layer "F.Cu") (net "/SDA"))
 (segment (start 123.43 91.523654) (end 123.43 92.476346) (width 0.2) (layer "F.Cu") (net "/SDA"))
 (segment (start 124.103654 93.15) (end 125.97 93.15) (width 0.2) (layer "F.Cu") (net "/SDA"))
 (segment (start 125.97 93.15) (end 127.12 92) (width 0.2) (layer "F.Cu") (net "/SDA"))
 (segment (start 155.018 84.3805) (end 158.62 80.7785) (width 0.2) (layer "B.Cu") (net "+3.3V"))
 (segment (start 132.2 92) (end 139.8195 84.3805) (width 0.2) (layer "B.Cu") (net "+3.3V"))
 (segment (start 139.8195 84.3805) (end 155.018 84.3805) (width 0.2) (layer "B.Cu") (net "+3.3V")))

